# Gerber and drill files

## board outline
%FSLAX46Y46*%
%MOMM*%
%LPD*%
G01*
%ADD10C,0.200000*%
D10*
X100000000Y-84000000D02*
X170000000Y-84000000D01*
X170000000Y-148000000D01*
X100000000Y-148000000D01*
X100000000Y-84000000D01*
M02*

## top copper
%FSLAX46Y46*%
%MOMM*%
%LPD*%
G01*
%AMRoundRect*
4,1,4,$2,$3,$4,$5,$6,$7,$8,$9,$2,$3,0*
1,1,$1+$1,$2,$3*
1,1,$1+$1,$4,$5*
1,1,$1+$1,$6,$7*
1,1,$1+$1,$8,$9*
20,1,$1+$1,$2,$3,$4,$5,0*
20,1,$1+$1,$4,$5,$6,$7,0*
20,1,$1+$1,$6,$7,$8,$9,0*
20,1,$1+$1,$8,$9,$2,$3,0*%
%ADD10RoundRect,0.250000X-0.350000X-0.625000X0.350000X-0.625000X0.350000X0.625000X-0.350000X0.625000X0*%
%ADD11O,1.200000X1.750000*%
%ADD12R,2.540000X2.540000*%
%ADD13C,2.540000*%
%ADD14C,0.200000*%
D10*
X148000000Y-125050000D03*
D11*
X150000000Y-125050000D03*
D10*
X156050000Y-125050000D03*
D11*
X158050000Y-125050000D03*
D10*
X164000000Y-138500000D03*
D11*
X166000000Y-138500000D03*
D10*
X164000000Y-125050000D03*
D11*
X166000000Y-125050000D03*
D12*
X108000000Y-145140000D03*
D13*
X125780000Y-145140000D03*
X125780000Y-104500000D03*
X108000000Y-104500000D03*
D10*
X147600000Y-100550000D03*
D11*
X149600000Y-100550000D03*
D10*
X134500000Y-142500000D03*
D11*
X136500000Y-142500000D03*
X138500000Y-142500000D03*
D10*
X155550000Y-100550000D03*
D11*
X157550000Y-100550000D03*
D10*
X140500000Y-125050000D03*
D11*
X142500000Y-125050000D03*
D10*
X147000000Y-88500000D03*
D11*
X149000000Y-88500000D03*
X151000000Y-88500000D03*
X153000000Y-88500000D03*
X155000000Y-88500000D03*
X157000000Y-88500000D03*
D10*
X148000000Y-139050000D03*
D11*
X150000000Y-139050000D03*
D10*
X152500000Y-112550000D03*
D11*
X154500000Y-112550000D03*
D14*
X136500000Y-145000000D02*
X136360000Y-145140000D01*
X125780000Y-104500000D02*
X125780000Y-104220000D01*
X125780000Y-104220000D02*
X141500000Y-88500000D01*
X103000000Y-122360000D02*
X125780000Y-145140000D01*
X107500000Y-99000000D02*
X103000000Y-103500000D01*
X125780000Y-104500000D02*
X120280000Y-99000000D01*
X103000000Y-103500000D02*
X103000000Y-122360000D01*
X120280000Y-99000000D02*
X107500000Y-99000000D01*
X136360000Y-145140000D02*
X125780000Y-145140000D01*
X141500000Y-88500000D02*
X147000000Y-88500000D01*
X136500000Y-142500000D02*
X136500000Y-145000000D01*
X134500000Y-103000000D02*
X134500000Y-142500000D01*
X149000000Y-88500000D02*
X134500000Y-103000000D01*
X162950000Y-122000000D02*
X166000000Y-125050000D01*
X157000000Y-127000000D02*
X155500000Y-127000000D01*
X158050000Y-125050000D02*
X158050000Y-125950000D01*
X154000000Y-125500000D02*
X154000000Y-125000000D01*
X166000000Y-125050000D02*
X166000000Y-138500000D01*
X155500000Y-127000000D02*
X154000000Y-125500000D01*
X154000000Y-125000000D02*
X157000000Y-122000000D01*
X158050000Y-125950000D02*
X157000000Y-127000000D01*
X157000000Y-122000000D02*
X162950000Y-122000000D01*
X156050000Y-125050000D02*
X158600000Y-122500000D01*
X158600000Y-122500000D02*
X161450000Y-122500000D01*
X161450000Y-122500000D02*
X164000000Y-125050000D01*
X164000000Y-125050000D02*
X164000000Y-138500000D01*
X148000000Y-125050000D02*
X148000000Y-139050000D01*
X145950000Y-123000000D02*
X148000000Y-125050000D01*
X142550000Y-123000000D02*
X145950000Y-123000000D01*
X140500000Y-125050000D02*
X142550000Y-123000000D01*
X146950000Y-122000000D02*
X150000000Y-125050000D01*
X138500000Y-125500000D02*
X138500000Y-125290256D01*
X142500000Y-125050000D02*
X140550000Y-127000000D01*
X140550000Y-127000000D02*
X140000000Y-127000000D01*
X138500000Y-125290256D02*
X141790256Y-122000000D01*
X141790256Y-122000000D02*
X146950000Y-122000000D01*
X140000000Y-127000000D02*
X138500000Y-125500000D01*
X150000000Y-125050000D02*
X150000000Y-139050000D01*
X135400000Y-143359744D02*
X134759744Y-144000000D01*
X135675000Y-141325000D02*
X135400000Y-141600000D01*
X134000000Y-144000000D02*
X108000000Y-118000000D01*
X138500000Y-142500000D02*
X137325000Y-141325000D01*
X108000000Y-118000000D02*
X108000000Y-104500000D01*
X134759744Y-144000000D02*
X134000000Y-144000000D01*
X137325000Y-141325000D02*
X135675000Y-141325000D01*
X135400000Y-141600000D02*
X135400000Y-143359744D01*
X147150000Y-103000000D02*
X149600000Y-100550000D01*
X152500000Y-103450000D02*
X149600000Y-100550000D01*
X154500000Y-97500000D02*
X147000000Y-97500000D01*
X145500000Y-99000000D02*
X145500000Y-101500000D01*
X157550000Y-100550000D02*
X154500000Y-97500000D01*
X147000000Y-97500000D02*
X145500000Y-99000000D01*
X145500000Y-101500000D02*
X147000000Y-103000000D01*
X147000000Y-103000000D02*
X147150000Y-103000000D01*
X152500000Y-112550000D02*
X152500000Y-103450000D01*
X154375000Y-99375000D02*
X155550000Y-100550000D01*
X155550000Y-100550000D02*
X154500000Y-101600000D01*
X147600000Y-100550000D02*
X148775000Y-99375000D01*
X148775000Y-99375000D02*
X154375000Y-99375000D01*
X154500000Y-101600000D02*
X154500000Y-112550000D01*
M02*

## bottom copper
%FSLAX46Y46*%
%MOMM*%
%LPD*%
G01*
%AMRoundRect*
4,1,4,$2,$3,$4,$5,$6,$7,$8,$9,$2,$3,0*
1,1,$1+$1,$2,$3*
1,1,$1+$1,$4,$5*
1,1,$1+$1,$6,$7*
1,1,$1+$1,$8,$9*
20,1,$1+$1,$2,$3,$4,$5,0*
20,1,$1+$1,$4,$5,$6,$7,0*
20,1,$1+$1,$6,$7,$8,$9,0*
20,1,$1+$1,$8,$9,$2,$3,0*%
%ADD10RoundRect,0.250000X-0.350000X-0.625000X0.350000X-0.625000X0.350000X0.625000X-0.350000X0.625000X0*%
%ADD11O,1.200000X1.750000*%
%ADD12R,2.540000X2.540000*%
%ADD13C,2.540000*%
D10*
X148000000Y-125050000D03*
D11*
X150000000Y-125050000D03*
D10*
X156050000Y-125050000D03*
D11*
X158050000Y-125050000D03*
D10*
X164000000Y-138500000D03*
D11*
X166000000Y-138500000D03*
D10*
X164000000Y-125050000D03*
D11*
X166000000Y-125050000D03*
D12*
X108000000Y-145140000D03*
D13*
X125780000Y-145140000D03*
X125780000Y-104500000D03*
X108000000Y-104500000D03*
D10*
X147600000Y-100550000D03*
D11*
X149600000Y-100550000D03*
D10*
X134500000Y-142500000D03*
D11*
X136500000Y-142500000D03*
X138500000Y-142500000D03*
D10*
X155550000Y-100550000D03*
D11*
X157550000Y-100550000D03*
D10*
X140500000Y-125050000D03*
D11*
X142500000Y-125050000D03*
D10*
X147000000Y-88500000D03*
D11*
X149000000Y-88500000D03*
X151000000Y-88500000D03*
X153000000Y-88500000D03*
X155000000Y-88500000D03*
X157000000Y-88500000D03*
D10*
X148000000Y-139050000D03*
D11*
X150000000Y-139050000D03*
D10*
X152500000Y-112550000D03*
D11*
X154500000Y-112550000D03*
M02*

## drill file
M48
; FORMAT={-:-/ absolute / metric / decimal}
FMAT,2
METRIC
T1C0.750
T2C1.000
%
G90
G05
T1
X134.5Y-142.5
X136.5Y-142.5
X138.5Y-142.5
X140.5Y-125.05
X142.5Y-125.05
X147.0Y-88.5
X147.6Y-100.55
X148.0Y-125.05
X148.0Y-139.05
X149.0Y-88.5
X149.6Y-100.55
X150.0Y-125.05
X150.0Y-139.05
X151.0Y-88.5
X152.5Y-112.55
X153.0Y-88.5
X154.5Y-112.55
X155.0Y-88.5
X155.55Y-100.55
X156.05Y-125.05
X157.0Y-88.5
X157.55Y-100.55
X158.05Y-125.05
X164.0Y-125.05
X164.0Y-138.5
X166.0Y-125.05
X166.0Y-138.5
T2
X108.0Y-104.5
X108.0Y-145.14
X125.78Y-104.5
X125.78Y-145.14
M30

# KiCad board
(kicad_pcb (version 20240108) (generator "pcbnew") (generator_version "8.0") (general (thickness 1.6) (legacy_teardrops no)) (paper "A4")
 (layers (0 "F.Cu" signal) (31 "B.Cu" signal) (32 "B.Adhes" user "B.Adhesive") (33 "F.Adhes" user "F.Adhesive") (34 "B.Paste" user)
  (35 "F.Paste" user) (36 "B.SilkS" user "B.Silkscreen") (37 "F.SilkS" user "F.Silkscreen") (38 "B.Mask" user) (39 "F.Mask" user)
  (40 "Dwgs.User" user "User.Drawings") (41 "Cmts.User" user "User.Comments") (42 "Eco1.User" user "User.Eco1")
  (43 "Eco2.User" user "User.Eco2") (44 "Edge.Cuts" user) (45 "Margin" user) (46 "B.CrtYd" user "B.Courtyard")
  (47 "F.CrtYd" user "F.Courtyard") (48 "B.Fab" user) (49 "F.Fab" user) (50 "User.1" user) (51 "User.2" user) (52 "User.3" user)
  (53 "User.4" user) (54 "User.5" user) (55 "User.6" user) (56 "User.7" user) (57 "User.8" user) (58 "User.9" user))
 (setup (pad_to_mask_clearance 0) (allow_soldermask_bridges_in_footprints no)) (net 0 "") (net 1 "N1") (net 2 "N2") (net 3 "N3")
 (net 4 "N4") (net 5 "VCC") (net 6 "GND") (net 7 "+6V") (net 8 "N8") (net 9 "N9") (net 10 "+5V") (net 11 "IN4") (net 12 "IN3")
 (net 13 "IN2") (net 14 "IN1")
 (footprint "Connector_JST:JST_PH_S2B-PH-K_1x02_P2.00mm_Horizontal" (layer "F.Cu") (at 148 125.05)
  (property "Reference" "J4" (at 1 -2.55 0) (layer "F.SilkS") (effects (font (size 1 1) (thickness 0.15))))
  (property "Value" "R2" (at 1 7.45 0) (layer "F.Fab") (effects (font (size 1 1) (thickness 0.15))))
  (pad "1" thru_hole roundrect (at 0 0) (size 1.2 1.75) (drill 0.75) (layers "*.Cu" "*.Mask") (remove_unused_layers no)
   (roundrect_rratio 0.208333) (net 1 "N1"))
  (pad "2" thru_hole oval (at 2 0) (size 1.2 1.75) (drill 0.75) (layers "*.Cu" "*.Mask") (remove_unused_layers no) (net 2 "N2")))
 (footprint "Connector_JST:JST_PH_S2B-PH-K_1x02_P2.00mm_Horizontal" (layer "F.Cu") (at 156.05 125.05)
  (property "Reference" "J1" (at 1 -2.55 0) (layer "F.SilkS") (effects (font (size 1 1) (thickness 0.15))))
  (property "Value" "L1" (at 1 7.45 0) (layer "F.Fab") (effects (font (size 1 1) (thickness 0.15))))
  (pad "1" thru_hole roundrect (at 0 0) (size 1.2 1.75) (drill 0.75) (layers "*.Cu" "*.Mask") (remove_unused_layers no)
   (roundrect_rratio 0.208333) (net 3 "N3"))
  (pad "2" thru_hole oval (at 2 0) (size 1.2 1.75) (drill 0.75) (layers "*.Cu" "*.Mask") (remove_unused_layers no) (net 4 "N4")))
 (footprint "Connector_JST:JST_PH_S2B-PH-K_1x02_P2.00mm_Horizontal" (layer "F.Cu") (at 164 138.5)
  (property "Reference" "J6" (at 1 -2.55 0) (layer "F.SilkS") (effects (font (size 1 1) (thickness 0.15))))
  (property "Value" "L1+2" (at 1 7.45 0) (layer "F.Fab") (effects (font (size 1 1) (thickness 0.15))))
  (pad "1" thru_hole roundrect (at 0 0) (size 1.2 1.75) (drill 0.75) (layers "*.Cu" "*.Mask") (remove_unused_layers no)
   (roundrect_rratio 0.208333) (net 3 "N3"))
  (pad "2" thru_hole oval (at 2 0) (size 1.2 1.75) (drill 0.75) (layers "*.Cu" "*.Mask") (remove_unused_layers no) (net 4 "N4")))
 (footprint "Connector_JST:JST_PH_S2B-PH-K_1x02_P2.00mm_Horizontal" (layer "F.Cu") (at 164 125.05)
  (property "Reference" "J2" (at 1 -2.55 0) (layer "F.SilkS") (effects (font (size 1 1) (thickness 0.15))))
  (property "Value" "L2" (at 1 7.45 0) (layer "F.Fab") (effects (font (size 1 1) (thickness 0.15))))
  (pad "1" thru_hole roundrect (at 0 0) (size 1.2 1.75) (drill 0.75) (layers "*.Cu" "*.Mask") (remove_unused_layers no)
   (roundrect_rratio 0.208333) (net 3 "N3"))
  (pad "2" thru_hole oval (at 2 0) (size 1.2 1.75) (drill 0.75) (layers "*.Cu" "*.Mask") (remove_unused_layers no) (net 4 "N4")))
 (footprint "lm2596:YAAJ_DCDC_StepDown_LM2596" (layer "F.Cu") (at 108 145.14 90)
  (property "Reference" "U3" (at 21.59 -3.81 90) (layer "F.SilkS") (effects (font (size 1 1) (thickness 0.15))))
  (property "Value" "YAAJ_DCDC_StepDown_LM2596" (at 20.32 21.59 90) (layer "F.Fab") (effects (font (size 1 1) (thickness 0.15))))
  (pad "1" thru_hole rect (at 0 0 90) (size 2.54 2.54) (drill 1) (layers "*.Cu" "*.Mask") (remove_unused_layers no) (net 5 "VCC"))
  (pad "2" thru_hole circle (at 0 17.78 90) (size 2.54 2.54) (drill 1) (layers "*.Cu" "*.Mask") (remove_unused_layers no) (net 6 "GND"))
  (pad "3" thru_hole circle (at 40.64 17.78 90) (size 2.54 2.54) (drill 1) (layers "*.Cu" "*.Mask") (remove_unused_layers no) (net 6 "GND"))
  (pad "4" thru_hole circle (at 40.64 0 90) (size 2.54 2.54) (drill 1) (layers "*.Cu" "*.Mask") (remove_unused_layers no) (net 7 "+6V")))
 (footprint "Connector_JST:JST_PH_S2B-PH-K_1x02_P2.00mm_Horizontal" (layer "F.Cu") (at 147.6 100.55)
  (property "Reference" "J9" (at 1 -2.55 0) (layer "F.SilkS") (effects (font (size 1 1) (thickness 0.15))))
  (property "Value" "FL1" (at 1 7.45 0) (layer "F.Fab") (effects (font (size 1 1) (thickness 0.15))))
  (pad "1" thru_hole roundrect (at 0 0) (size 1.2 1.75) (drill 0.75) (layers "*.Cu" "*.Mask") (remove_unused_layers no)
   (roundrect_rratio 0.208333) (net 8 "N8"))
  (pad "2" thru_hole oval (at 2 0) (size 1.2 1.75) (drill 0.75) (layers "*.Cu" "*.Mask") (remove_unused_layers no) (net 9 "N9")))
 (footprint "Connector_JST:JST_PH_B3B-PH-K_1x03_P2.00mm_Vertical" (layer "F.Cu") (at 134.5 142.5)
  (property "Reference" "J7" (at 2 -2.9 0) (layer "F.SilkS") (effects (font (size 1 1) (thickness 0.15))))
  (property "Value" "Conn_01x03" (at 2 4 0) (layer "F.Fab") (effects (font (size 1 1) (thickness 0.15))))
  (pad "1" thru_hole roundrect (at 0 0) (size 1.2 1.75) (drill 0.75) (layers "*.Cu" "*.Mask") (remove_unused_layers no)
   (roundrect_rratio 0.208333) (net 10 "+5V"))
  (pad "2" thru_hole oval (at 2 0) (size 1.2 1.75) (drill 0.75) (layers "*.Cu" "*.Mask") (remove_unused_layers no) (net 6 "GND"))
  (pad "3" thru_hole oval (at 4 0) (size 1.2 1.75) (drill 0.75) (layers "*.Cu" "*.Mask") (remove_unused_layers no) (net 7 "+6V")))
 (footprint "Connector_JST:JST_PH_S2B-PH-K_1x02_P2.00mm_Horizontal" (layer "F.Cu") (at 155.55 100.55)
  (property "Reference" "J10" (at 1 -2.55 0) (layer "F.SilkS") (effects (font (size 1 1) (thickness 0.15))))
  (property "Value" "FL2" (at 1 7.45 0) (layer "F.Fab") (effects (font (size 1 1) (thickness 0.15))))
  (pad "1" thru_hole roundrect (at 0 0) (size 1.2 1.75) (drill 0.75) (layers "*.Cu" "*.Mask") (remove_unused_layers no)
   (roundrect_rratio 0.208333) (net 8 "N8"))
  (pad "2" thru_hole oval (at 2 0) (size 1.2 1.75) (drill 0.75) (layers "*.Cu" "*.Mask") (remove_unused_layers no) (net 9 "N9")))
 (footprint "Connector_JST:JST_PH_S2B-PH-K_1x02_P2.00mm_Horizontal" (layer "F.Cu") (at 140.5 125.05)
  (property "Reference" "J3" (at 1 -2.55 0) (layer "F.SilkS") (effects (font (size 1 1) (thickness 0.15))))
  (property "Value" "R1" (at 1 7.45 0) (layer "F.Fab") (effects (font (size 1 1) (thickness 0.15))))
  (pad "1" thru_hole roundrect (at 0 0) (size 1.2 1.75) (drill 0.75) (layers "*.Cu" "*.Mask") (remove_unused_layers no)
   (roundrect_rratio 0.208333) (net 1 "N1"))
  (pad "2" thru_hole oval (at 2 0) (size 1.2 1.75) (drill 0.75) (layers "*.Cu" "*.Mask") (remove_unused_layers no) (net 2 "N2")))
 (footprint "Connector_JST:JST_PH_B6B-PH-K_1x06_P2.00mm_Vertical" (layer "F.Cu") (at 147 88.5)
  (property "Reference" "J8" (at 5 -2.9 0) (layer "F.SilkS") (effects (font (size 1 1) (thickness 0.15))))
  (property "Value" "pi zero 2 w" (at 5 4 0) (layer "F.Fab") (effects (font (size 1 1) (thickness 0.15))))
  (pad "1" thru_hole roundrect (at 0 0) (size 1.2 1.75) (drill 0.75) (layers "*.Cu" "*.Mask") (remove_unused_layers no)
   (roundrect_rratio 0.208333) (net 6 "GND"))
  (pad "2" thru_hole oval (at 2 0) (size 1.2 1.75) (drill 0.75) (layers "*.Cu" "*.Mask") (remove_unused_layers no) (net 10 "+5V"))
  (pad "3" thru_hole oval (at 4 0) (size 1.2 1.75) (drill 0.75) (layers "*.Cu" "*.Mask") (remove_unused_layers no) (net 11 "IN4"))
  (pad "4" thru_hole oval (at 6 0) (size 1.2 1.75) (drill 0.75) (layers "*.Cu" "*.Mask") (remove_unused_layers no) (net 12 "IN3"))
  (pad "5" thru_hole oval (at 8 0) (size 1.2 1.75) (drill 0.75) (layers "*.Cu" "*.Mask") (remove_unused_layers no) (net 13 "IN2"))
  (pad "6" thru_hole oval (at 10 0) (size 1.2 1.75) (drill 0.75) (layers "*.Cu" "*.Mask") (remove_unused_layers no) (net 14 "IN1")))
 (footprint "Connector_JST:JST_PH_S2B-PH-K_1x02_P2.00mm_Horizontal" (layer "F.Cu") (at 148 139.05)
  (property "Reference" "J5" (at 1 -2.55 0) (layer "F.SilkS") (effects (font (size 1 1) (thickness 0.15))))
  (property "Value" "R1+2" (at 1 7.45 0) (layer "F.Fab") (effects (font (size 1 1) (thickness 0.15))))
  (pad "1" thru_hole roundrect (at 0 0) (size 1.2 1.75) (drill 0.75) (layers "*.Cu" "*.Mask") (remove_unused_layers no)
   (roundrect_rratio 0.208333) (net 1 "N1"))
  (pad "2" thru_hole oval (at 2 0) (size 1.2 1.75) (drill 0.75) (layers "*.Cu" "*.Mask") (remove_unused_layers no) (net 2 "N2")))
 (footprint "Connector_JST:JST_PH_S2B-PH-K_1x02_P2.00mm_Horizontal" (layer "F.Cu") (at 152.5 112.55)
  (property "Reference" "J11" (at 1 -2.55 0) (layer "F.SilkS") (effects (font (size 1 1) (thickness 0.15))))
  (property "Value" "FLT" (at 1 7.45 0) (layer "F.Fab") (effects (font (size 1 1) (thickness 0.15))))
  (pad "1" thru_hole roundrect (at 0 0) (size 1.2 1.75) (drill 0.75) (layers "*.Cu" "*.Mask") (remove_unused_layers no)
   (roundrect_rratio 0.208333) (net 9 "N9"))
  (pad "2" thru_hole oval (at 2 0) (size 1.2 1.75) (drill 0.75) (layers "*.Cu" "*.Mask") (remove_unused_layers no) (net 8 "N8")))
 (gr_rect (start 100 84) (end 170 148) (stroke (width 0.2) (type default)) (fill none) (layer "Edge.Cuts"))
 (segment (start 136.5 145) (end 136.36 145.14) (width 0.2) (layer "F.Cu") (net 6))
 (segment (start 125.78 104.5) (end 125.78 104.22) (width 0.2) (layer "F.Cu") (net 6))
 (segment (start 125.78 104.22) (end 141.5 88.5) (width 0.2) (layer "F.Cu") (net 6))
 (segment (start 103 122.36) (end 125.78 145.14) (width 0.2) (layer "F.Cu") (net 6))
 (segment (start 107.5 99) (end 103 103.5) (width 0.2) (layer "F.Cu") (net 6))
 (segment (start 125.78 104.5) (end 120.28 99) (width 0.2) (layer "F.Cu") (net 6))
 (segment (start 103 103.5) (end 103 122.36) (width 0.2) (layer "F.Cu") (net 6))
 (segment (start 120.28 99) (end 107.5 99) (width 0.2) (layer "F.Cu") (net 6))
 (segment (start 136.36 145.14) (end 125.78 145.14) (width 0.2) (layer "F.Cu") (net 6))
 (segment (start 141.5 88.5) (end 147 88.5) (width 0.2) (layer "F.Cu") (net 6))
 (segment (start 136.5 142.5) (end 136.5 145) (width 0.2) (layer "F.Cu") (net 6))
 (segment (start 134.5 103) (end 134.5 142.5) (width 0.2) (layer "F.Cu") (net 10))
 (segment (start 149 88.5) (end 134.5 103) (width 0.2) (layer "F.Cu") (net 10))
 (segment (start 162.95 122) (end 166 125.05) (width 0.2) (layer "F.Cu") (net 4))
 (segment (start 157 127) (end 155.5 127) (width 0.2) (layer "F.Cu") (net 4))
 (segment (start 158.05 125.05) (end 158.05 125.95) (width 0.2) (layer "F.Cu") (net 4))
 (segment (start 154 125.5) (end 154 125) (width 0.2) (layer "F.Cu") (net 4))
 (segment (start 166 125.05) (end 166 138.5) (width 0.2) (layer "F.Cu") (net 4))
 (segment (start 155.5 127) (end 154 125.5) (width 0.2) (layer "F.Cu") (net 4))
 (segment (start 154 125) (end 157 122) (width 0.2) (layer "F.Cu") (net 4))
 (segment (start 158.05 125.95) (end 157 127) (width 0.2) (layer "F.Cu") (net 4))
 (segment (start 157 122) (end 162.95 122) (width 0.2) (layer "F.Cu") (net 4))
 (segment (start 156.05 125.05) (end 158.6 122.5) (width 0.2) (layer "F.Cu") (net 3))
 (segment (start 158.6 122.5) (end 161.45 122.5) (width 0.2) (layer "F.Cu") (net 3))
 (segment (start 161.45 122.5) (end 164 125.05) (width 0.2) (layer "F.Cu") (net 3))
 (segment (start 164 125.05) (end 164 138.5) (width 0.2) (layer "F.Cu") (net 3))
 (segment (start 148 125.05) (end 148 139.05) (width 0.2) (layer "F.Cu") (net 1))
 (segment (start 145.95 123) (end 148 125.05) (width 0.2) (layer "F.Cu") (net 1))
 (segment (start 142.55 123) (end 145.95 123) (width 0.2) (layer "F.Cu") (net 1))
 (segment (start 140.5 125.05) (end 142.55 123) (width 0.2) (layer "F.Cu") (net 1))
 (segment (start 146.95 122) (end 150 125.05) (width 0.2) (layer "F.Cu") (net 2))
 (segment (start 138.5 125.5) (end 138.5 125.290256) (width 0.2) (layer "F.Cu") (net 2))
 (segment (start 142.5 125.05) (end 140.55 127) (width 0.2) (layer "F.Cu") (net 2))
 (segment (start 140.55 127) (end 140 127) (width 0.2) (layer "F.Cu") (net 2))
 (segment (start 138.5 125.290256) (end 141.790256 122) (width 0.2) (layer "F.Cu") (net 2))
 (segment (start 141.790256 122) (end 146.95 122) (width 0.2) (layer "F.Cu") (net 2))
 (segment (start 140 127) (end 138.5 125.5) (width 0.2) (layer "F.Cu") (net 2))
 (segment (start 150 125.05) (end 150 139.05) (width 0.2) (layer "F.Cu") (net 2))
 (segment (start 135.4 143.359744) (end 134.759744 144) (width 0.2) (layer "F.Cu") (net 7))
 (segment (start 135.675 141.325) (end 135.4 141.6) (width 0.2) (layer "F.Cu") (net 7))
 (segment (start 134 144) (end 108 118) (width 0.2) (layer "F.Cu") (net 7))
 (segment (start 138.5 142.5) (end 137.325 141.325) (width 0.2) (layer "F.Cu") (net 7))
 (segment (start 108 118) (end 108 104.5) (width 0.2) (layer "F.Cu") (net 7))
 (segment (start 134.759744 144) (end 134 144) (width 0.2) (layer "F.Cu") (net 7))
 (segment (start 137.325 141.325) (end 135.675 141.325) (width 0.2) (layer "F.Cu") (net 7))
 (segment (start 135.4 141.6) (end 135.4 143.359744) (width 0.2) (layer "F.Cu") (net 7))
 (segment (start 147.15 103) (end 149.6 100.55) (width 0.2) (layer "F.Cu") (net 9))
 (segment (start 152.5 103.45) (end 149.6 100.55) (width 0.2) (layer "F.Cu") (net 9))
 (segment (start 154.5 97.5) (end 147 97.5) (width 0.2) (layer "F.Cu") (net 9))
 (segment (start 145.5 99) (end 145.5 101.5) (width 0.2) (layer "F.Cu") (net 9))
 (segment (start 157.55 100.55) (end 154.5 97.5) (width 0.2) (layer "F.Cu") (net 9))
 (segment (start 147 97.5) (end 145.5 99) (width 0.2) (layer "F.Cu") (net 9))
 (segment (start 145.5 101.5) (end 147 103) (width 0.2) (layer "F.Cu") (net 9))
 (segment (start 147 103) (end 147.15 103) (width 0.2) (layer "F.Cu") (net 9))
 (segment (start 152.5 112.55) (end 152.5 103.45) (width 0.2) (layer "F.Cu") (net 9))
 (segment (start 154.375 99.375) (end 155.55 100.55) (width 0.2) (layer "F.Cu") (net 8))
 (segment (start 155.55 100.55) (end 154.5 101.6) (width 0.2) (layer "F.Cu") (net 8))
 (segment (start 147.6 100.55) (end 148.775 99.375) (width 0.2) (layer "F.Cu") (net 8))
 (segment (start 148.775 99.375) (end 154.375 99.375) (width 0.2) (layer "F.Cu") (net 8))
 (segment (start 154.5 101.6) (end 154.5 112.55) (width 0.2) (layer "F.Cu") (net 8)))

